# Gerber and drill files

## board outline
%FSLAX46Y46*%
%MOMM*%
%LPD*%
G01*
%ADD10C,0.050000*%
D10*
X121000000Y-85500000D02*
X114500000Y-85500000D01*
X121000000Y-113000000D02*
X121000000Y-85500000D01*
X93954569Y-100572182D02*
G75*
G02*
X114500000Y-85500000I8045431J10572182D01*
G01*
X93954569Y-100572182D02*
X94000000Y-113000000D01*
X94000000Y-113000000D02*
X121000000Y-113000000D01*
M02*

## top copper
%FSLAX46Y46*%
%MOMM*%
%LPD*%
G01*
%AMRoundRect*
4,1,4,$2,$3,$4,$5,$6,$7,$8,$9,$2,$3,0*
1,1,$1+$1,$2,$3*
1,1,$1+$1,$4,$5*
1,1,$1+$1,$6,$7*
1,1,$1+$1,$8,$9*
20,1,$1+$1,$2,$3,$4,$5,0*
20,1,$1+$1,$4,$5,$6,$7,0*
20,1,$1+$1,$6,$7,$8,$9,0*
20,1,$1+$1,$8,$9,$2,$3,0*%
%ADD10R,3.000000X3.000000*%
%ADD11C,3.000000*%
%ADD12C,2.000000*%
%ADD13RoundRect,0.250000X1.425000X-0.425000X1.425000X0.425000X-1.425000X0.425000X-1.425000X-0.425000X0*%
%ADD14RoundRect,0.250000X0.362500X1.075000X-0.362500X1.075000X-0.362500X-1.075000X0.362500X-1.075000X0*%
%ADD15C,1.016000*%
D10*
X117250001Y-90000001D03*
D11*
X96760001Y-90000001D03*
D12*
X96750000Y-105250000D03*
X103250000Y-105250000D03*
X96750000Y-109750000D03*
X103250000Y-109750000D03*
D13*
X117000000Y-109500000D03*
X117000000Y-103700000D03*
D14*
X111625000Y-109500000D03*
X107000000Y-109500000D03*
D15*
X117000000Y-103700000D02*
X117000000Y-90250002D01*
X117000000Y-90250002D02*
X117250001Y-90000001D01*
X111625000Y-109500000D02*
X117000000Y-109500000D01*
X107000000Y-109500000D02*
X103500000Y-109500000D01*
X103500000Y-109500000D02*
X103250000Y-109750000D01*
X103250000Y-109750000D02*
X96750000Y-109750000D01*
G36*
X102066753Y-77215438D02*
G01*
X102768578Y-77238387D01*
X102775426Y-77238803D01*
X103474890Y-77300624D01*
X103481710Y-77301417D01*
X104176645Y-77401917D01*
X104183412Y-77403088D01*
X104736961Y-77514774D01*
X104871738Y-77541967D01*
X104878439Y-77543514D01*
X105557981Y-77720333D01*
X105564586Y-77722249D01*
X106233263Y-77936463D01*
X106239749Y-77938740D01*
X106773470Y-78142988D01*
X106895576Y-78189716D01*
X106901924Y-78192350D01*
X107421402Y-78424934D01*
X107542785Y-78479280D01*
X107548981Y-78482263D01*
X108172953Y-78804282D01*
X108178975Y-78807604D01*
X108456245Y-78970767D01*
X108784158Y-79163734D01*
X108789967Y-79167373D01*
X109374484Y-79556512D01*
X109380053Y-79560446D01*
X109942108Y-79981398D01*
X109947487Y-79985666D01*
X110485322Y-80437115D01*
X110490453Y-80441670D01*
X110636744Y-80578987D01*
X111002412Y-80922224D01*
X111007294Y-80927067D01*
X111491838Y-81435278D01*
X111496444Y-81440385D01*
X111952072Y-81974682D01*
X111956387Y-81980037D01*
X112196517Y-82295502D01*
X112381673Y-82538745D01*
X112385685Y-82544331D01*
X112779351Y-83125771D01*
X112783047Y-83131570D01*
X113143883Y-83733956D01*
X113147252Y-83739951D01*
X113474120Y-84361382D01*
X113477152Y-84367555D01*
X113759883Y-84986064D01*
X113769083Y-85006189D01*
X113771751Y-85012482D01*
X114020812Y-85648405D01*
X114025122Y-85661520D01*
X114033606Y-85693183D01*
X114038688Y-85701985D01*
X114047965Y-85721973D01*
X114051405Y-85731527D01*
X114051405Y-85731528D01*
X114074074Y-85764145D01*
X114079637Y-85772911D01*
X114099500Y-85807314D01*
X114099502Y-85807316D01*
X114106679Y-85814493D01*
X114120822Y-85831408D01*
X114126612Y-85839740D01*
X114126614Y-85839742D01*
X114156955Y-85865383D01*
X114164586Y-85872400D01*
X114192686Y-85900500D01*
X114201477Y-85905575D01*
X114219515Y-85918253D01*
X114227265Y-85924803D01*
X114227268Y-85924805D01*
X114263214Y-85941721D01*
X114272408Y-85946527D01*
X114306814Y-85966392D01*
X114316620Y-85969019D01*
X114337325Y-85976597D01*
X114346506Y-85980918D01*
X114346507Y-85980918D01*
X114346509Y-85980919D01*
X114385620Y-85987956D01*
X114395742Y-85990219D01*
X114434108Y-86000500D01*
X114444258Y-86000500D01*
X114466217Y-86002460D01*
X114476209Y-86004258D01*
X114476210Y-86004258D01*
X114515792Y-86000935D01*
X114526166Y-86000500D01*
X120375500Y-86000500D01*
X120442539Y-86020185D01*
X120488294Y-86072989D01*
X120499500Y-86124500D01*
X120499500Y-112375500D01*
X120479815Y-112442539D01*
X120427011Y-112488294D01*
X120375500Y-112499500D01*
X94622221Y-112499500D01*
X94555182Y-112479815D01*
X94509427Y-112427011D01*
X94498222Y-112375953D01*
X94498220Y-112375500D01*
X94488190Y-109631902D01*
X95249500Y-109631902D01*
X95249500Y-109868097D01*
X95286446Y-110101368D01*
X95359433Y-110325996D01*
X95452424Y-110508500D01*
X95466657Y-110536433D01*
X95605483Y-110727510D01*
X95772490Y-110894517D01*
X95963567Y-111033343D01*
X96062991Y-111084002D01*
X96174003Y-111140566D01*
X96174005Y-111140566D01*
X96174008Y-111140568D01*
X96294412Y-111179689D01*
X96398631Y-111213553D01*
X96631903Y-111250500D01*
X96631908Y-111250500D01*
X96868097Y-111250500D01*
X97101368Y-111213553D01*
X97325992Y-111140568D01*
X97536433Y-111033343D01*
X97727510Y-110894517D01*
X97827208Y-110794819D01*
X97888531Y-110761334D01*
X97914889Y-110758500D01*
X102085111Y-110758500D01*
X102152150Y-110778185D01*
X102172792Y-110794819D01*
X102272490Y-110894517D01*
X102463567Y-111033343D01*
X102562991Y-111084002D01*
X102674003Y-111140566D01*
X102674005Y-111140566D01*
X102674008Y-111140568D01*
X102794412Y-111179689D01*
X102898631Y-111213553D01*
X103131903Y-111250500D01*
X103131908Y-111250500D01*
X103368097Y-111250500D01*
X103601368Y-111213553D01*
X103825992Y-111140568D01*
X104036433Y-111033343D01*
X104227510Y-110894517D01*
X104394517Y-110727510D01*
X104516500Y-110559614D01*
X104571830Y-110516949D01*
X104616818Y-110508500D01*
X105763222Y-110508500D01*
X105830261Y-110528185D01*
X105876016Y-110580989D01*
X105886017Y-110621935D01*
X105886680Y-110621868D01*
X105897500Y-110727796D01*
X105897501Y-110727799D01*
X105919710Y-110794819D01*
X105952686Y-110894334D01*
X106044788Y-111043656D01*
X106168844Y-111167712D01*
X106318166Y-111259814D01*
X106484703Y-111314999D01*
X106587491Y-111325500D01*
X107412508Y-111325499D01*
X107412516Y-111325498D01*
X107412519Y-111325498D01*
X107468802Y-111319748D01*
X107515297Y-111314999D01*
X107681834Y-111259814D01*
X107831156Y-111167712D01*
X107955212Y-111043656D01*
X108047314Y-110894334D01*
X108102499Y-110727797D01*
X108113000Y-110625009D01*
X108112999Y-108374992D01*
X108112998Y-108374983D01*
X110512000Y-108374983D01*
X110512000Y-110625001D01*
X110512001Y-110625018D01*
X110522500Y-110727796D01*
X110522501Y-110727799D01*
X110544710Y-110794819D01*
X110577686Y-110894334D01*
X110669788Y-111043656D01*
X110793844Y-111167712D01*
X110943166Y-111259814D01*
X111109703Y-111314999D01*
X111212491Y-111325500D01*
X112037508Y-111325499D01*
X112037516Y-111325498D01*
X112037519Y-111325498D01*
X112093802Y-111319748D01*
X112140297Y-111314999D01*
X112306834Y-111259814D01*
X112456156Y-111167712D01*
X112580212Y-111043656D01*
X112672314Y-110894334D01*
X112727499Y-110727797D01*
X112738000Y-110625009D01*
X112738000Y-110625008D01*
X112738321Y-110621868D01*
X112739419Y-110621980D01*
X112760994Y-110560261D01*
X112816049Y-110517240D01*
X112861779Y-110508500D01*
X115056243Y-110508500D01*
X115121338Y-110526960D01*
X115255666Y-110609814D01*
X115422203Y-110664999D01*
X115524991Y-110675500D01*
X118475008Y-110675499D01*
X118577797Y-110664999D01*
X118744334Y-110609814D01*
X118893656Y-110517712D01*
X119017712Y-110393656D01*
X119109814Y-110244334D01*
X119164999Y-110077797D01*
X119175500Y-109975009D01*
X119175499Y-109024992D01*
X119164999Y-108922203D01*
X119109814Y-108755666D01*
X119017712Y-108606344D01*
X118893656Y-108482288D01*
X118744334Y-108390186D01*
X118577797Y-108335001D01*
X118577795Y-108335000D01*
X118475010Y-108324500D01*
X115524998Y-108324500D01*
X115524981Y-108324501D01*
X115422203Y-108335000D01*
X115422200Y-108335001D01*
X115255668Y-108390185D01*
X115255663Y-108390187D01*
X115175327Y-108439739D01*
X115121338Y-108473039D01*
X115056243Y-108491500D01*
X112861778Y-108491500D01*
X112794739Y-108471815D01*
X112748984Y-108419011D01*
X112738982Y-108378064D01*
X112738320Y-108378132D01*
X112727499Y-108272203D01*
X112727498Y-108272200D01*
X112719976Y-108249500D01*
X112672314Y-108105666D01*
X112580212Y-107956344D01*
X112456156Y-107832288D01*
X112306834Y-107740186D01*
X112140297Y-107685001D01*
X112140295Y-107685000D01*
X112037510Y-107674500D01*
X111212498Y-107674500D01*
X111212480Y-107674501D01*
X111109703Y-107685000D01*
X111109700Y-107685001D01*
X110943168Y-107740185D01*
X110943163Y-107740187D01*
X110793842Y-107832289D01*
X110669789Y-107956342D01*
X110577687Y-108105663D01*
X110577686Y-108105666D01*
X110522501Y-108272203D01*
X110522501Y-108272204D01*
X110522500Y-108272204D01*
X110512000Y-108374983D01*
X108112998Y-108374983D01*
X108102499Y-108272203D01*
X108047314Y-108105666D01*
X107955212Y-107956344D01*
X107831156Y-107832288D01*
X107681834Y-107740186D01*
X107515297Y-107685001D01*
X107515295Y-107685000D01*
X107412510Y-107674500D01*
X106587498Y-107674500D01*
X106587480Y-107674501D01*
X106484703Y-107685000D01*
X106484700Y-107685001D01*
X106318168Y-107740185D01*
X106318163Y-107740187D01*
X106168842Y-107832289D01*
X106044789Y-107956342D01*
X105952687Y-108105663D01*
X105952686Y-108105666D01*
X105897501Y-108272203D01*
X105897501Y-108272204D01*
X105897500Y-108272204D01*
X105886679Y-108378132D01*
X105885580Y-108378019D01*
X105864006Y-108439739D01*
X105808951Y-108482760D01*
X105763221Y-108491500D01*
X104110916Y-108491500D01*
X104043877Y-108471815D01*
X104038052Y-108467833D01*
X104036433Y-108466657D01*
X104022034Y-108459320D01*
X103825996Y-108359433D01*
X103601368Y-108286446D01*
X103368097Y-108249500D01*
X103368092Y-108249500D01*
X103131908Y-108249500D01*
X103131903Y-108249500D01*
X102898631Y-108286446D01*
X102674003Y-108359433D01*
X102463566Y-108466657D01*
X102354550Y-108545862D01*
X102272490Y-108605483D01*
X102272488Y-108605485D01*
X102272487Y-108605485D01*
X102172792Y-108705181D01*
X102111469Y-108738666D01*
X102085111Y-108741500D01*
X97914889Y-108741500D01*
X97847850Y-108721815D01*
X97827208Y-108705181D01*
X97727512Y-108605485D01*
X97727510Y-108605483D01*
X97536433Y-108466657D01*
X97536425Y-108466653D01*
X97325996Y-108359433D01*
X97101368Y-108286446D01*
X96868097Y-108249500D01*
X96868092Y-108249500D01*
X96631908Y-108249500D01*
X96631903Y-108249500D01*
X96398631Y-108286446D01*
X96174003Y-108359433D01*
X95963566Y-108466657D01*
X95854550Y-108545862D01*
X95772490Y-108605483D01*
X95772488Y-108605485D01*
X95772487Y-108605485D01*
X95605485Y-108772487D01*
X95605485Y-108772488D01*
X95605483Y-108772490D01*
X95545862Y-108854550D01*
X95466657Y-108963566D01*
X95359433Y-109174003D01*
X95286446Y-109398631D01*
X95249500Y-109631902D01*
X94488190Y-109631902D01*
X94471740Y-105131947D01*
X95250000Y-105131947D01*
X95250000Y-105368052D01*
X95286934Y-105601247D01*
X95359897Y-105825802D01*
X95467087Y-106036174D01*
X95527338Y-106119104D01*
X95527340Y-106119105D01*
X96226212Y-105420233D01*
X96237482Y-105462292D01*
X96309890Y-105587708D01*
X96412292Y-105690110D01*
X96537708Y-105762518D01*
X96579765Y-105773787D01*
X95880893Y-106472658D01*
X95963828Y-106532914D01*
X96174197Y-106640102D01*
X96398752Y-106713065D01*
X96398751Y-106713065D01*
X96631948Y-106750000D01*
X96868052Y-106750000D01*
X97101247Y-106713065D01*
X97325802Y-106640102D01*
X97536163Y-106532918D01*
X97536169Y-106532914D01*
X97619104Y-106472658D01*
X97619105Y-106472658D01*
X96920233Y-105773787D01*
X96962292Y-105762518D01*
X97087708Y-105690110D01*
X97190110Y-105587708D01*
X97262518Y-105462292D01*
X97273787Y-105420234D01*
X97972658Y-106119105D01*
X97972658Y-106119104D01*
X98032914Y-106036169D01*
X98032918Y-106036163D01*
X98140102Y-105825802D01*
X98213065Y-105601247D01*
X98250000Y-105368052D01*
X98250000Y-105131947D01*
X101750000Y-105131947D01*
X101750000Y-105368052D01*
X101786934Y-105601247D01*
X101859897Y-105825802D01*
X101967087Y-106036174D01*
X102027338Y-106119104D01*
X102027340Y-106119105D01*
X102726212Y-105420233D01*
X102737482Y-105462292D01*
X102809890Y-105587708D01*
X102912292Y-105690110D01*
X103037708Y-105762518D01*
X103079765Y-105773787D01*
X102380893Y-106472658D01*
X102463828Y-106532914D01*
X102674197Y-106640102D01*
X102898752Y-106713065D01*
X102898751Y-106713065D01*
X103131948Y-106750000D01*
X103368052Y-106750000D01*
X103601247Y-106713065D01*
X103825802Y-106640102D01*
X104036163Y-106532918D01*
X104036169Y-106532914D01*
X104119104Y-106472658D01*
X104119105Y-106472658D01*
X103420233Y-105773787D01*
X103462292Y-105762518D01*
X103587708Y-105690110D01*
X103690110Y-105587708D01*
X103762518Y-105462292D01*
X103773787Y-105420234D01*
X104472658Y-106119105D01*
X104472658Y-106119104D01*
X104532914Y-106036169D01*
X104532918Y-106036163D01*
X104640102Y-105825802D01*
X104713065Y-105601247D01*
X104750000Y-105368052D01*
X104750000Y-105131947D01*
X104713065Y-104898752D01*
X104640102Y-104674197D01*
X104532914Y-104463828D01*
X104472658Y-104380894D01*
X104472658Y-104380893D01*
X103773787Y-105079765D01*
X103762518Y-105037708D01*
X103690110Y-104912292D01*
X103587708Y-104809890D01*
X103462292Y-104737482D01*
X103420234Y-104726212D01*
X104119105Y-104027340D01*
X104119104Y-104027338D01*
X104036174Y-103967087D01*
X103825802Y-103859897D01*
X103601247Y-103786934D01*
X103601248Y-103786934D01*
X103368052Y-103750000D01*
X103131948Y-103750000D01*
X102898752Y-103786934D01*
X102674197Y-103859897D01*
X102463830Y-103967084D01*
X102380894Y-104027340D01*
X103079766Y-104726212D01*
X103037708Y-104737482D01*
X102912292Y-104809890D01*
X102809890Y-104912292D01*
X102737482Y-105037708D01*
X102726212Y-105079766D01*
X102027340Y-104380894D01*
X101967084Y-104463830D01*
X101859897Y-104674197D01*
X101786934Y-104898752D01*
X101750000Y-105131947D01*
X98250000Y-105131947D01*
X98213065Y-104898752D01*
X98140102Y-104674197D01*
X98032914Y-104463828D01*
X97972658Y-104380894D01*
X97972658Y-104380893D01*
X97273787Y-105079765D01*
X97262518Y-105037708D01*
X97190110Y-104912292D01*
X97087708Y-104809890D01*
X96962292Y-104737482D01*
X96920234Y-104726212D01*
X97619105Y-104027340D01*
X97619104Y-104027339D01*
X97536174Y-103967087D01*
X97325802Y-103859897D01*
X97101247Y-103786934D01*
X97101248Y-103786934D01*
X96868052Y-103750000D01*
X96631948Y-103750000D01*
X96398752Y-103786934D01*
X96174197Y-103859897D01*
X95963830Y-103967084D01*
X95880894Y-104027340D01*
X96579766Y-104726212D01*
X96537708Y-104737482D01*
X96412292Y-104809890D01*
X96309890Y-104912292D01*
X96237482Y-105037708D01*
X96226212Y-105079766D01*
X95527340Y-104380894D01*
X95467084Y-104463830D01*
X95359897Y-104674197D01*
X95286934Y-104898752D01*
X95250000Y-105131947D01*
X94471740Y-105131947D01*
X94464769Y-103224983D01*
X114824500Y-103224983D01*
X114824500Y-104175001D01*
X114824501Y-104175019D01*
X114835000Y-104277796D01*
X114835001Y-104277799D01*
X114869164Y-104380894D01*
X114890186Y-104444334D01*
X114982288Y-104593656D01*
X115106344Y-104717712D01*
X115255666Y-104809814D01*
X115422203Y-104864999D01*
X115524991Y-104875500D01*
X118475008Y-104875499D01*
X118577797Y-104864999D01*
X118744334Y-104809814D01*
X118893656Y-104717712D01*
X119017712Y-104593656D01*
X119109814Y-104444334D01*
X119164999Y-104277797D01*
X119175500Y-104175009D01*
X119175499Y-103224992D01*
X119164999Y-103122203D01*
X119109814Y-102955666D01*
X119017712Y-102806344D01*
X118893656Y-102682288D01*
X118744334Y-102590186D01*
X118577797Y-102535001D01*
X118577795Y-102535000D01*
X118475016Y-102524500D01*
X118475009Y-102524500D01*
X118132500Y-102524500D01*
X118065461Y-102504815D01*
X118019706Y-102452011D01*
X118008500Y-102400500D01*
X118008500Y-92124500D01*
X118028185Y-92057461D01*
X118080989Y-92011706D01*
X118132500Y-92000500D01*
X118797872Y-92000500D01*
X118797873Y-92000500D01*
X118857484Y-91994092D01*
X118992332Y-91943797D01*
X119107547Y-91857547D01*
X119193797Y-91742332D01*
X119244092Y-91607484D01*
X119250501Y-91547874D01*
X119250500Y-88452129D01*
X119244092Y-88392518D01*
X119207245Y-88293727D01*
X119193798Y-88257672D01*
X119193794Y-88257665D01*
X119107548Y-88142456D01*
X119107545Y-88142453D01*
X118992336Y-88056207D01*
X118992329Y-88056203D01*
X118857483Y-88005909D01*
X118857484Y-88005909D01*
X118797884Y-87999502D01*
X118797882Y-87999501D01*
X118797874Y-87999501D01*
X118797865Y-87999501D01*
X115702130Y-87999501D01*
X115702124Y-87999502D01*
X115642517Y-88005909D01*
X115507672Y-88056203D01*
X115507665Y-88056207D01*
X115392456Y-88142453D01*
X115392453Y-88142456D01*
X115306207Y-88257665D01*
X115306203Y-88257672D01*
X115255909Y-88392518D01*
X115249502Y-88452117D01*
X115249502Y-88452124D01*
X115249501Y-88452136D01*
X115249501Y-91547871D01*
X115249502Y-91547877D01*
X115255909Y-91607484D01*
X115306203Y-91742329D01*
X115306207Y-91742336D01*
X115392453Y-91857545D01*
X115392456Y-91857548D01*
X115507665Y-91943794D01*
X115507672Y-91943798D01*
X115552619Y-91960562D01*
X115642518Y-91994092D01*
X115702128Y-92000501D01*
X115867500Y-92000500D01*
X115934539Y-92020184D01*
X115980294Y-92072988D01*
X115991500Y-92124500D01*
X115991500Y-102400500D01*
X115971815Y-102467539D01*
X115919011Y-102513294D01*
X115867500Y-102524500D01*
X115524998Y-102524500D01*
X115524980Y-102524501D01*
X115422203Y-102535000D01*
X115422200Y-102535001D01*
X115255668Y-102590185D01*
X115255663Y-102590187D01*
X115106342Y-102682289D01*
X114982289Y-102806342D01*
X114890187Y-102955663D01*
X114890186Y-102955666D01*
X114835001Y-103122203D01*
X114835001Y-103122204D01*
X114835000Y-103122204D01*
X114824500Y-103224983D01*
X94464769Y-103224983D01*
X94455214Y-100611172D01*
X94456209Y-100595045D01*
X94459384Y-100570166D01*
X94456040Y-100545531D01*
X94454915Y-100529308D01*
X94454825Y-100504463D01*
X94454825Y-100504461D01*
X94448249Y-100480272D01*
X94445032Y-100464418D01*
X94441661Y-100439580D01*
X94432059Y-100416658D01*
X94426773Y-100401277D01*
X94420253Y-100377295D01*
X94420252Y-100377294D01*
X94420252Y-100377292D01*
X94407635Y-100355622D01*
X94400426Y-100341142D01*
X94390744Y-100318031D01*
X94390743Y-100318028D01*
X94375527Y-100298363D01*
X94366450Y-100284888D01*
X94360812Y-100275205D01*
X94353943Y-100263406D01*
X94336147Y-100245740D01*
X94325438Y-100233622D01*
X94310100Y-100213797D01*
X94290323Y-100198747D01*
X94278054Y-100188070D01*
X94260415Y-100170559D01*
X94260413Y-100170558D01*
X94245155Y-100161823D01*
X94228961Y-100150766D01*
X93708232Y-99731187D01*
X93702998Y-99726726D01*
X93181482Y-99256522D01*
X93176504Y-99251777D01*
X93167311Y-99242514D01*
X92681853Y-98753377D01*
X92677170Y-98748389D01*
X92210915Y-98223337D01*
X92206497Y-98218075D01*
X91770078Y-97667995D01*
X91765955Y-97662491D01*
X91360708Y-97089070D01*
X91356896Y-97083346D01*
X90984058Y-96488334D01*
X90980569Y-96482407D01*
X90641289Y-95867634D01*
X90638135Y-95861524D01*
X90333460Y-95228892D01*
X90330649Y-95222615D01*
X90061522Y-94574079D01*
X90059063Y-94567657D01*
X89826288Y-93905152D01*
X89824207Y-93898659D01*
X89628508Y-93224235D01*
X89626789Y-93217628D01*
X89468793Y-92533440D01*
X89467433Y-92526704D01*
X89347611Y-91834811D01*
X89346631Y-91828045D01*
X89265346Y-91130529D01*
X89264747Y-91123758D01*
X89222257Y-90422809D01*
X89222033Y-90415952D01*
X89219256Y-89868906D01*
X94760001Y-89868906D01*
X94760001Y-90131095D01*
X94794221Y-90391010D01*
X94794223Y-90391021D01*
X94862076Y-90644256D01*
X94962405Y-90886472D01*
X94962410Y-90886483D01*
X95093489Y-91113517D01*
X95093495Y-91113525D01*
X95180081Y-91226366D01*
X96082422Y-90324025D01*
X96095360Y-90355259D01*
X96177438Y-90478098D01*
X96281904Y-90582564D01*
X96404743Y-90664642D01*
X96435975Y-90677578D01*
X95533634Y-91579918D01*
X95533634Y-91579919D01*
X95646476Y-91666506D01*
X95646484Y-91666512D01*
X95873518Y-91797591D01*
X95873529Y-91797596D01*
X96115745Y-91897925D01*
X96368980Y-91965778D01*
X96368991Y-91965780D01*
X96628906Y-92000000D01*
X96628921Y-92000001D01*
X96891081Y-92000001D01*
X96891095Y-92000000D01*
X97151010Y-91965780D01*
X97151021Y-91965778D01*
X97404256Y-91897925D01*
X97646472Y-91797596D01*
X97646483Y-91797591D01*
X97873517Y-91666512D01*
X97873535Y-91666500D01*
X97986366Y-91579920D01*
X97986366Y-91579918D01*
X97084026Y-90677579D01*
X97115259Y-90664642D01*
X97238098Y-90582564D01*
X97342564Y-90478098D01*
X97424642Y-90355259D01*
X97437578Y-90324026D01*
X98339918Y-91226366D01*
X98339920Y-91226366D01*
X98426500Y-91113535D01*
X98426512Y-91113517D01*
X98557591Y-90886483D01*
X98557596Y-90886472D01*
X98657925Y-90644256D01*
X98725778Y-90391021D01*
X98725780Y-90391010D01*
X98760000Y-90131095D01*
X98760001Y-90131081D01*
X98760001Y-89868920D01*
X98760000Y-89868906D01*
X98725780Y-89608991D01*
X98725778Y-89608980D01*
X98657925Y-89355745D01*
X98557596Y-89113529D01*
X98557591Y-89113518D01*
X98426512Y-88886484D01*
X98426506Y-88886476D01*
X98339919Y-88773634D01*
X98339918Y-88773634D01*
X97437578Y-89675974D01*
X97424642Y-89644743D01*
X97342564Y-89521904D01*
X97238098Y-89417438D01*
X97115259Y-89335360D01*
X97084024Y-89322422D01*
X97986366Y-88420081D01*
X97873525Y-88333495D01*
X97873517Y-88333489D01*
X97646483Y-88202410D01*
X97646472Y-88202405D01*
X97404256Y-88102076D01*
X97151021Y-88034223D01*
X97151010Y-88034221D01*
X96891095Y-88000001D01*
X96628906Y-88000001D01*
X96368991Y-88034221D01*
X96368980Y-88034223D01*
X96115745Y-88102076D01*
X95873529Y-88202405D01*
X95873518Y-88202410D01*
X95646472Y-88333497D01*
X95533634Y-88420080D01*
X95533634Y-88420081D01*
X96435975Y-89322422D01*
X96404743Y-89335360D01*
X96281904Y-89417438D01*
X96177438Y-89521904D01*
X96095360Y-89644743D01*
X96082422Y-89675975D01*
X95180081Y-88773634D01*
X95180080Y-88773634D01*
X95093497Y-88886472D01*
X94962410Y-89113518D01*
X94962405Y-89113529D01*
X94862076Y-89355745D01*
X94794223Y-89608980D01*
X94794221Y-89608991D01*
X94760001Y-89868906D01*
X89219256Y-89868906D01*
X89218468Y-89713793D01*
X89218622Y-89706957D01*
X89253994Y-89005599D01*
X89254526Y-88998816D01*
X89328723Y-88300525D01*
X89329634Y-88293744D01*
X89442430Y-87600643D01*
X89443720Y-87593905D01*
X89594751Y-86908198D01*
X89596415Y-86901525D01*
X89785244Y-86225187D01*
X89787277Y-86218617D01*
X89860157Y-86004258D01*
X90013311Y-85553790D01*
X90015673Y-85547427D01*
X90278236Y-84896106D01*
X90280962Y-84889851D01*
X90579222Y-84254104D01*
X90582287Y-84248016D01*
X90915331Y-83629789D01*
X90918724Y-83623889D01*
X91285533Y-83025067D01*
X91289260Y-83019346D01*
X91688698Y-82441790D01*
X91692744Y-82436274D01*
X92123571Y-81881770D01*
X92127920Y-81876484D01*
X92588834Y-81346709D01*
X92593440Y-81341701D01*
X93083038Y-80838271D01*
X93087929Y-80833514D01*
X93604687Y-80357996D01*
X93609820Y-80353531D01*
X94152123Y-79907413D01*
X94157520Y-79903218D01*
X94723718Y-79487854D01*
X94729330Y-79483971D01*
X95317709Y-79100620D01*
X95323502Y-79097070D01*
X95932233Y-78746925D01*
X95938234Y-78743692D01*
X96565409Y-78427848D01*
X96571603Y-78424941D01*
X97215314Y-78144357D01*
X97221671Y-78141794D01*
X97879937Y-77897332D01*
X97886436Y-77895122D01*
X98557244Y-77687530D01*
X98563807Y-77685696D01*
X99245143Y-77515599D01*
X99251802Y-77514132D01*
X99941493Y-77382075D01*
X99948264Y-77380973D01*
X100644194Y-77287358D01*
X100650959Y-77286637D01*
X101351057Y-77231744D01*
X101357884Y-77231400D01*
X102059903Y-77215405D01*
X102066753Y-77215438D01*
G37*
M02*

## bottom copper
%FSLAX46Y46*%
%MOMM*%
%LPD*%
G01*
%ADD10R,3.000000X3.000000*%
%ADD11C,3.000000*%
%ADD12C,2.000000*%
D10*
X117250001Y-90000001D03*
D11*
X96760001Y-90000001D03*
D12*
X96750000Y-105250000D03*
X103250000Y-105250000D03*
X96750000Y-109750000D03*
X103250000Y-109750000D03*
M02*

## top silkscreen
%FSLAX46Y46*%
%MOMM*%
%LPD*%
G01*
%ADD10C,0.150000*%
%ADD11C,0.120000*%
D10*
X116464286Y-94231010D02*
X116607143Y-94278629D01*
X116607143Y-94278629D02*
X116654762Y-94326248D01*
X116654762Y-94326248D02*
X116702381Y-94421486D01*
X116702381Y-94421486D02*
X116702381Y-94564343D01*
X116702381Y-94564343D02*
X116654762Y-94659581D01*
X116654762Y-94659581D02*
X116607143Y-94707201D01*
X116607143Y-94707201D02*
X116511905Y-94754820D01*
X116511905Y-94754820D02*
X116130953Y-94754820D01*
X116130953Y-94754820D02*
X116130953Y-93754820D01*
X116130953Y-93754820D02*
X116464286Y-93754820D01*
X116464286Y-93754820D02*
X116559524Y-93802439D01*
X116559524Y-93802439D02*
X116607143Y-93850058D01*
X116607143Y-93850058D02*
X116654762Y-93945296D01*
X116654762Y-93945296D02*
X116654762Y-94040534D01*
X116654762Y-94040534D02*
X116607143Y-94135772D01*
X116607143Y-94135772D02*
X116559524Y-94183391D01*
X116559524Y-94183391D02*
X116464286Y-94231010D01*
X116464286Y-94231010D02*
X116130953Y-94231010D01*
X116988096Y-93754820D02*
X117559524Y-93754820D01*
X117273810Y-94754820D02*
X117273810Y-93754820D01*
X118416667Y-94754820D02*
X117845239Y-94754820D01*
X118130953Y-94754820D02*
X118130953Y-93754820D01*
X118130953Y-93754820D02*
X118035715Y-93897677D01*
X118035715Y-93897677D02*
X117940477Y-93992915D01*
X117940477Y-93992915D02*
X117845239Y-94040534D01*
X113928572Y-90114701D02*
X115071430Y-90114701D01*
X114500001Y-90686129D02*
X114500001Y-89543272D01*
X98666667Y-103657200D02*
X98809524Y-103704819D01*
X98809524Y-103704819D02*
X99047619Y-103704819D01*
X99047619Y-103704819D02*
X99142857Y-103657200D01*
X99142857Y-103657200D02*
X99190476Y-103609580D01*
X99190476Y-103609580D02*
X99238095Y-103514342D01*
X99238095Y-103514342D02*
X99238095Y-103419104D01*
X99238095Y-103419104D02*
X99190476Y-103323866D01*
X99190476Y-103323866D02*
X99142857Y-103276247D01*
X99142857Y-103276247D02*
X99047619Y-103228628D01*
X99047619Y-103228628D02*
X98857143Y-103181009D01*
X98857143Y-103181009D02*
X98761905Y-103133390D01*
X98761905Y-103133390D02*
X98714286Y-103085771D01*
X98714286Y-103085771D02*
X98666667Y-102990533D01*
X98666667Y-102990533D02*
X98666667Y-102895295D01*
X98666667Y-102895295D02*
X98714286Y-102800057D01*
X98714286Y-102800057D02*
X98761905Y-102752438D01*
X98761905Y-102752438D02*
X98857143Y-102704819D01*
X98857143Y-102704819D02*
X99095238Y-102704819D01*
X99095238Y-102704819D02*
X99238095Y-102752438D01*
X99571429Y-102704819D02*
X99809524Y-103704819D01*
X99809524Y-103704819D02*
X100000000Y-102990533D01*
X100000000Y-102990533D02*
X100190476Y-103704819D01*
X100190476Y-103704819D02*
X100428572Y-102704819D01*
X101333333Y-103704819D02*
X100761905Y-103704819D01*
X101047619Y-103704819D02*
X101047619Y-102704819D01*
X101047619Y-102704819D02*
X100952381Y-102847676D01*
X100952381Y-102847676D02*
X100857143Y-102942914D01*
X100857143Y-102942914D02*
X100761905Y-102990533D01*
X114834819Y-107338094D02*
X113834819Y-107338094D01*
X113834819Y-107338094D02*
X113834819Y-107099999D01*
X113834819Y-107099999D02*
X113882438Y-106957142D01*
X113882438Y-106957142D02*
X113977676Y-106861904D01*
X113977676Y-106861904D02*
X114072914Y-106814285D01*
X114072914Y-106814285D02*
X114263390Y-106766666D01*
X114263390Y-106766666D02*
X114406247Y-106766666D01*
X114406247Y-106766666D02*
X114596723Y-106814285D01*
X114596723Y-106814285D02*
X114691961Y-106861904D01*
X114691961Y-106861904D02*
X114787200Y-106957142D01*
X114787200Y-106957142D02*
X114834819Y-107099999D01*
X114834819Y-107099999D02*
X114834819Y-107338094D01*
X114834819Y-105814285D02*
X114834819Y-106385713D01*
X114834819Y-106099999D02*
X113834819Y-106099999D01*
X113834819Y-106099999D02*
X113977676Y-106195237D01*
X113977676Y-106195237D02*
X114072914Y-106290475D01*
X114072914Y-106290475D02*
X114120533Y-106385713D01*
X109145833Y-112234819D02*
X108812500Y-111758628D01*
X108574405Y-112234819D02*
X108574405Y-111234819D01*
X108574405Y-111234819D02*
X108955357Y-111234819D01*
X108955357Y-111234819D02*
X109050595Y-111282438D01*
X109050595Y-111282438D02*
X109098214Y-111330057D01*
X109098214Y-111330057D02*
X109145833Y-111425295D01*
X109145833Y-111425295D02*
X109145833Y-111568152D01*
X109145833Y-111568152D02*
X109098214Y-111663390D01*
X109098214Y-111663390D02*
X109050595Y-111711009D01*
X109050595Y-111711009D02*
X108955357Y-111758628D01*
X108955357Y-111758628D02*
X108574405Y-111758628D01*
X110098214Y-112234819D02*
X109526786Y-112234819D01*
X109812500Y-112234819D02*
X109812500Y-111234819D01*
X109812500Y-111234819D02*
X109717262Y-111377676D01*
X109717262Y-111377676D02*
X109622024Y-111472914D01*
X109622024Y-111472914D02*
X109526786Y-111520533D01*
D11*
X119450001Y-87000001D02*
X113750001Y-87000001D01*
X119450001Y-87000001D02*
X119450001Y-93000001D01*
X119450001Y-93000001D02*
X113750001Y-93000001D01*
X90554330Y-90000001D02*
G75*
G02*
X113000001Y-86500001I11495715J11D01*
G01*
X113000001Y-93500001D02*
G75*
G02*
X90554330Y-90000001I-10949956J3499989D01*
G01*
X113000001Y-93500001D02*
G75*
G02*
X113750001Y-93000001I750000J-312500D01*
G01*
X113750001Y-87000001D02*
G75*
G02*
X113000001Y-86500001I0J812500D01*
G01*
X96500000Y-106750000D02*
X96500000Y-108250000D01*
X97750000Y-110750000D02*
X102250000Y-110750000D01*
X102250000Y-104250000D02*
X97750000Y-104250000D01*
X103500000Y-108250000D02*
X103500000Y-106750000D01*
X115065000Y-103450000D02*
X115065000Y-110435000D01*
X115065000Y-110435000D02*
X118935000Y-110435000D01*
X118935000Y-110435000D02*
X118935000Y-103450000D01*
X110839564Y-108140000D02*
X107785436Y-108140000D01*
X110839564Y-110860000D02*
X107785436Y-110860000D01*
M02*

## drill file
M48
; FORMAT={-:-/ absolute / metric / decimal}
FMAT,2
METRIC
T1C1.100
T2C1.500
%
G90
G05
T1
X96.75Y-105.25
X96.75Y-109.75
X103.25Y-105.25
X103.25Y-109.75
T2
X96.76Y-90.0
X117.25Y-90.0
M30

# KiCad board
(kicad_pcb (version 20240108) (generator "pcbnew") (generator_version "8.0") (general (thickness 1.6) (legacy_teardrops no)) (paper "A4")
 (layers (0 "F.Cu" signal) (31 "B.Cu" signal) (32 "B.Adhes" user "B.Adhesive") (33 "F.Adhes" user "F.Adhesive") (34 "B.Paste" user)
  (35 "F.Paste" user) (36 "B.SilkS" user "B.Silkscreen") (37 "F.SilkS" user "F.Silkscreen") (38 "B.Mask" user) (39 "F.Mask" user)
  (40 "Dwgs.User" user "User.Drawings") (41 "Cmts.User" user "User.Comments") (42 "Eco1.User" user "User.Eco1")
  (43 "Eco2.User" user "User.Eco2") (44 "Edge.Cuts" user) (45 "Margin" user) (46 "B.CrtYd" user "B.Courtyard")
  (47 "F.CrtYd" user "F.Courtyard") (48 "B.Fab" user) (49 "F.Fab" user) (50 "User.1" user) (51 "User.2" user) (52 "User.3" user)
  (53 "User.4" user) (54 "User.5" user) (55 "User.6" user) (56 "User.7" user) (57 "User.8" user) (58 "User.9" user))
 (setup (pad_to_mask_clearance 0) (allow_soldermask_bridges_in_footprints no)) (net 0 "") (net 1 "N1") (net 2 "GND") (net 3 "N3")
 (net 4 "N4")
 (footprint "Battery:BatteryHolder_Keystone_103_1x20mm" (layer "F.Cu") (at 117.250001 90.000001 180)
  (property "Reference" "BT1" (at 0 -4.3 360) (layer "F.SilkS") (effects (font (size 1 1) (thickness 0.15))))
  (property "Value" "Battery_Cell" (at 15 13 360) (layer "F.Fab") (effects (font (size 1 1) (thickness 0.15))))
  (fp_line (start -2.2 3) (end 3.5 3) (stroke (width 0.12) (type solid)) (layer "F.SilkS"))
  (fp_line (start -2.2 3) (end -2.2 -3) (stroke (width 0.12) (type solid)) (layer "F.SilkS"))
  (fp_line (start -2.2 -3) (end 3.5 -3) (stroke (width 0.12) (type solid)) (layer "F.SilkS"))
  (fp_arc (start 26.695671 0) (mid 16.971103 11.358466) (end 4.25 3.5) (stroke (width 0.12) (type solid)) (layer "F.SilkS"))
  (fp_arc (start 4.25 -3.5) (mid 16.971103 -11.358466) (end 26.695671 0) (stroke (width 0.12) (type solid)) (layer "F.SilkS"))
  (fp_arc (start 4.25 -3.5) (mid 3.950694 -3.136459) (end 3.5 -3) (stroke (width 0.12) (type solid)) (layer "F.SilkS"))
  (fp_arc (start 3.5 3) (mid 3.950694 3.136459) (end 4.25 3.5) (stroke (width 0.12) (type solid)) (layer "F.SilkS"))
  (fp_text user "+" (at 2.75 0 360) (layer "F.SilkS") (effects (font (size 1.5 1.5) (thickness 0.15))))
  (pad "1" thru_hole rect (at 0 0 180) (size 3 3) (drill 1.5) (layers "*.Cu" "*.Mask") (remove_unused_layers no) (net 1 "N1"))
  (pad "2" thru_hole circle (at 20.49 0 180) (size 3 3) (drill 1.5) (layers "*.Cu" "*.Mask") (remove_unused_layers no) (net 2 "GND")))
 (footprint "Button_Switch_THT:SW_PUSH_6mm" (layer "F.Cu") (at 96.75 105.25)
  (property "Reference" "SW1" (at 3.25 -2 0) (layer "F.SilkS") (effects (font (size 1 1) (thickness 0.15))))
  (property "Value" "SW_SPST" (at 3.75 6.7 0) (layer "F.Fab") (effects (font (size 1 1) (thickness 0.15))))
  (fp_line (start -0.25 1.5) (end -0.25 3) (stroke (width 0.12) (type solid)) (layer "F.SilkS"))
  (fp_line (start 1 5.5) (end 5.5 5.5) (stroke (width 0.12) (type solid)) (layer "F.SilkS"))
  (fp_line (start 5.5 -1) (end 1 -1) (stroke (width 0.12) (type solid)) (layer "F.SilkS"))
  (fp_line (start 6.75 3) (end 6.75 1.5) (stroke (width 0.12) (type solid)) (layer "F.SilkS"))
  (pad "1" thru_hole circle (at 0 0 90) (size 2 2) (drill 1.1) (layers "*.Cu" "*.Mask") (remove_unused_layers no) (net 2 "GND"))
  (pad "1" thru_hole circle (at 6.5 0 90) (size 2 2) (drill 1.1) (layers "*.Cu" "*.Mask") (remove_unused_layers no) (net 2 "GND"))
  (pad "2" thru_hole circle (at 0 4.5 90) (size 2 2) (drill 1.1) (layers "*.Cu" "*.Mask") (remove_unused_layers no) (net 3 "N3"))
  (pad "2" thru_hole circle (at 6.5 4.5 90) (size 2 2) (drill 1.1) (layers "*.Cu" "*.Mask") (remove_unused_layers no) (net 3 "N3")))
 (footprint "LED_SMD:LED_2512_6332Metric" (layer "F.Cu") (at 117 106.6 90)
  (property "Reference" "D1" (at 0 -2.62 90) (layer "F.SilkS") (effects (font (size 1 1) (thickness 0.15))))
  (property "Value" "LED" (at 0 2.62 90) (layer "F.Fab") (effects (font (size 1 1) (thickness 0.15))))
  (fp_line (start 3.15 -1.935) (end -3.835 -1.935) (stroke (width 0.12) (type solid)) (layer "F.SilkS"))
  (fp_line (start -3.835 -1.935) (end -3.835 1.935) (stroke (width 0.12) (type solid)) (layer "F.SilkS"))
  (fp_line (start -3.835 1.935) (end 3.15 1.935) (stroke (width 0.12) (type solid)) (layer "F.SilkS"))
  (pad "1" smd roundrect (at -2.9 0 90) (size 1.35 3.35) (layers "F.Cu" "F.Paste" "F.Mask") (roundrect_rratio 0.185185) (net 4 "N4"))
  (pad "2" smd roundrect (at 2.9 0 90) (size 1.35 3.35) (layers "F.Cu" "F.Paste" "F.Mask") (roundrect_rratio 0.185185) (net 1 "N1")))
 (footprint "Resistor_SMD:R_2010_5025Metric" (layer "F.Cu") (at 109.3125 109.5 180)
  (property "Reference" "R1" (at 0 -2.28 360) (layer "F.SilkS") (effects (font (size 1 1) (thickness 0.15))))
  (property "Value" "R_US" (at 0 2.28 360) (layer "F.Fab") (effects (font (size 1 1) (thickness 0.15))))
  (fp_line (start -1.527064 1.36) (end 1.527064 1.36) (stroke (width 0.12) (type solid)) (layer "F.SilkS"))
  (fp_line (start -1.527064 -1.36) (end 1.527064 -1.36) (stroke (width 0.12) (type solid)) (layer "F.SilkS"))
  (pad "1" smd roundrect (at -2.3125 0 180) (size 1.225 2.65) (layers "F.Cu" "F.Paste" "F.Mask") (roundrect_rratio 0.204082) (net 4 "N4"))
  (pad "2" smd roundrect (at 2.3125 0 180) (size 1.225 2.65) (layers "F.Cu" "F.Paste" "F.Mask") (roundrect_rratio 0.204082) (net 3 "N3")))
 (gr_line (start 121 85.5) (end 114.5 85.5) (stroke (width 0.05) (type default)) (layer "Edge.Cuts"))
 (gr_line (start 121 113) (end 121 85.5) (stroke (width 0.05) (type default)) (layer "Edge.Cuts"))
 (gr_arc (start 93.954569 100.572182) (mid 94.141663 79.288019) (end 114.5 85.5) (stroke (width 0.05) (type default)) (layer "Edge.Cuts"))
 (gr_line (start 93.954569 100.572182) (end 94 113) (stroke (width 0.05) (type default)) (layer "Edge.Cuts"))
 (gr_line (start 94 113) (end 121 113) (stroke (width 0.05) (type default)) (layer "Edge.Cuts"))
 (segment (start 117 103.7) (end 117 90.250002) (width 1.016) (layer "F.Cu") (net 1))
 (segment (start 117 90.250002) (end 117.250001 90.000001) (width 1.016) (layer "F.Cu") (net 1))
 (segment (start 111.625 109.5) (end 117 109.5) (width 1.016) (layer "F.Cu") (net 4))
 (segment (start 107 109.5) (end 103.5 109.5) (width 1.016) (layer "F.Cu") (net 3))
 (segment (start 103.5 109.5) (end 103.25 109.75) (width 1.016) (layer "F.Cu") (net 3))
 (segment (start 103.25 109.75) (end 96.75 109.75) (width 1.016) (layer "F.Cu") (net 3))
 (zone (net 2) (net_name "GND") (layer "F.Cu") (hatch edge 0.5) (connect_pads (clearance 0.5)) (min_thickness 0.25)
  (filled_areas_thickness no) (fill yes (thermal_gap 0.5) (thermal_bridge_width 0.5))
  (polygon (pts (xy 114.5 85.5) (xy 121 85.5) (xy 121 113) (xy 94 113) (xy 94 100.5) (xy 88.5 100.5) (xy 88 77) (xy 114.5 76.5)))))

